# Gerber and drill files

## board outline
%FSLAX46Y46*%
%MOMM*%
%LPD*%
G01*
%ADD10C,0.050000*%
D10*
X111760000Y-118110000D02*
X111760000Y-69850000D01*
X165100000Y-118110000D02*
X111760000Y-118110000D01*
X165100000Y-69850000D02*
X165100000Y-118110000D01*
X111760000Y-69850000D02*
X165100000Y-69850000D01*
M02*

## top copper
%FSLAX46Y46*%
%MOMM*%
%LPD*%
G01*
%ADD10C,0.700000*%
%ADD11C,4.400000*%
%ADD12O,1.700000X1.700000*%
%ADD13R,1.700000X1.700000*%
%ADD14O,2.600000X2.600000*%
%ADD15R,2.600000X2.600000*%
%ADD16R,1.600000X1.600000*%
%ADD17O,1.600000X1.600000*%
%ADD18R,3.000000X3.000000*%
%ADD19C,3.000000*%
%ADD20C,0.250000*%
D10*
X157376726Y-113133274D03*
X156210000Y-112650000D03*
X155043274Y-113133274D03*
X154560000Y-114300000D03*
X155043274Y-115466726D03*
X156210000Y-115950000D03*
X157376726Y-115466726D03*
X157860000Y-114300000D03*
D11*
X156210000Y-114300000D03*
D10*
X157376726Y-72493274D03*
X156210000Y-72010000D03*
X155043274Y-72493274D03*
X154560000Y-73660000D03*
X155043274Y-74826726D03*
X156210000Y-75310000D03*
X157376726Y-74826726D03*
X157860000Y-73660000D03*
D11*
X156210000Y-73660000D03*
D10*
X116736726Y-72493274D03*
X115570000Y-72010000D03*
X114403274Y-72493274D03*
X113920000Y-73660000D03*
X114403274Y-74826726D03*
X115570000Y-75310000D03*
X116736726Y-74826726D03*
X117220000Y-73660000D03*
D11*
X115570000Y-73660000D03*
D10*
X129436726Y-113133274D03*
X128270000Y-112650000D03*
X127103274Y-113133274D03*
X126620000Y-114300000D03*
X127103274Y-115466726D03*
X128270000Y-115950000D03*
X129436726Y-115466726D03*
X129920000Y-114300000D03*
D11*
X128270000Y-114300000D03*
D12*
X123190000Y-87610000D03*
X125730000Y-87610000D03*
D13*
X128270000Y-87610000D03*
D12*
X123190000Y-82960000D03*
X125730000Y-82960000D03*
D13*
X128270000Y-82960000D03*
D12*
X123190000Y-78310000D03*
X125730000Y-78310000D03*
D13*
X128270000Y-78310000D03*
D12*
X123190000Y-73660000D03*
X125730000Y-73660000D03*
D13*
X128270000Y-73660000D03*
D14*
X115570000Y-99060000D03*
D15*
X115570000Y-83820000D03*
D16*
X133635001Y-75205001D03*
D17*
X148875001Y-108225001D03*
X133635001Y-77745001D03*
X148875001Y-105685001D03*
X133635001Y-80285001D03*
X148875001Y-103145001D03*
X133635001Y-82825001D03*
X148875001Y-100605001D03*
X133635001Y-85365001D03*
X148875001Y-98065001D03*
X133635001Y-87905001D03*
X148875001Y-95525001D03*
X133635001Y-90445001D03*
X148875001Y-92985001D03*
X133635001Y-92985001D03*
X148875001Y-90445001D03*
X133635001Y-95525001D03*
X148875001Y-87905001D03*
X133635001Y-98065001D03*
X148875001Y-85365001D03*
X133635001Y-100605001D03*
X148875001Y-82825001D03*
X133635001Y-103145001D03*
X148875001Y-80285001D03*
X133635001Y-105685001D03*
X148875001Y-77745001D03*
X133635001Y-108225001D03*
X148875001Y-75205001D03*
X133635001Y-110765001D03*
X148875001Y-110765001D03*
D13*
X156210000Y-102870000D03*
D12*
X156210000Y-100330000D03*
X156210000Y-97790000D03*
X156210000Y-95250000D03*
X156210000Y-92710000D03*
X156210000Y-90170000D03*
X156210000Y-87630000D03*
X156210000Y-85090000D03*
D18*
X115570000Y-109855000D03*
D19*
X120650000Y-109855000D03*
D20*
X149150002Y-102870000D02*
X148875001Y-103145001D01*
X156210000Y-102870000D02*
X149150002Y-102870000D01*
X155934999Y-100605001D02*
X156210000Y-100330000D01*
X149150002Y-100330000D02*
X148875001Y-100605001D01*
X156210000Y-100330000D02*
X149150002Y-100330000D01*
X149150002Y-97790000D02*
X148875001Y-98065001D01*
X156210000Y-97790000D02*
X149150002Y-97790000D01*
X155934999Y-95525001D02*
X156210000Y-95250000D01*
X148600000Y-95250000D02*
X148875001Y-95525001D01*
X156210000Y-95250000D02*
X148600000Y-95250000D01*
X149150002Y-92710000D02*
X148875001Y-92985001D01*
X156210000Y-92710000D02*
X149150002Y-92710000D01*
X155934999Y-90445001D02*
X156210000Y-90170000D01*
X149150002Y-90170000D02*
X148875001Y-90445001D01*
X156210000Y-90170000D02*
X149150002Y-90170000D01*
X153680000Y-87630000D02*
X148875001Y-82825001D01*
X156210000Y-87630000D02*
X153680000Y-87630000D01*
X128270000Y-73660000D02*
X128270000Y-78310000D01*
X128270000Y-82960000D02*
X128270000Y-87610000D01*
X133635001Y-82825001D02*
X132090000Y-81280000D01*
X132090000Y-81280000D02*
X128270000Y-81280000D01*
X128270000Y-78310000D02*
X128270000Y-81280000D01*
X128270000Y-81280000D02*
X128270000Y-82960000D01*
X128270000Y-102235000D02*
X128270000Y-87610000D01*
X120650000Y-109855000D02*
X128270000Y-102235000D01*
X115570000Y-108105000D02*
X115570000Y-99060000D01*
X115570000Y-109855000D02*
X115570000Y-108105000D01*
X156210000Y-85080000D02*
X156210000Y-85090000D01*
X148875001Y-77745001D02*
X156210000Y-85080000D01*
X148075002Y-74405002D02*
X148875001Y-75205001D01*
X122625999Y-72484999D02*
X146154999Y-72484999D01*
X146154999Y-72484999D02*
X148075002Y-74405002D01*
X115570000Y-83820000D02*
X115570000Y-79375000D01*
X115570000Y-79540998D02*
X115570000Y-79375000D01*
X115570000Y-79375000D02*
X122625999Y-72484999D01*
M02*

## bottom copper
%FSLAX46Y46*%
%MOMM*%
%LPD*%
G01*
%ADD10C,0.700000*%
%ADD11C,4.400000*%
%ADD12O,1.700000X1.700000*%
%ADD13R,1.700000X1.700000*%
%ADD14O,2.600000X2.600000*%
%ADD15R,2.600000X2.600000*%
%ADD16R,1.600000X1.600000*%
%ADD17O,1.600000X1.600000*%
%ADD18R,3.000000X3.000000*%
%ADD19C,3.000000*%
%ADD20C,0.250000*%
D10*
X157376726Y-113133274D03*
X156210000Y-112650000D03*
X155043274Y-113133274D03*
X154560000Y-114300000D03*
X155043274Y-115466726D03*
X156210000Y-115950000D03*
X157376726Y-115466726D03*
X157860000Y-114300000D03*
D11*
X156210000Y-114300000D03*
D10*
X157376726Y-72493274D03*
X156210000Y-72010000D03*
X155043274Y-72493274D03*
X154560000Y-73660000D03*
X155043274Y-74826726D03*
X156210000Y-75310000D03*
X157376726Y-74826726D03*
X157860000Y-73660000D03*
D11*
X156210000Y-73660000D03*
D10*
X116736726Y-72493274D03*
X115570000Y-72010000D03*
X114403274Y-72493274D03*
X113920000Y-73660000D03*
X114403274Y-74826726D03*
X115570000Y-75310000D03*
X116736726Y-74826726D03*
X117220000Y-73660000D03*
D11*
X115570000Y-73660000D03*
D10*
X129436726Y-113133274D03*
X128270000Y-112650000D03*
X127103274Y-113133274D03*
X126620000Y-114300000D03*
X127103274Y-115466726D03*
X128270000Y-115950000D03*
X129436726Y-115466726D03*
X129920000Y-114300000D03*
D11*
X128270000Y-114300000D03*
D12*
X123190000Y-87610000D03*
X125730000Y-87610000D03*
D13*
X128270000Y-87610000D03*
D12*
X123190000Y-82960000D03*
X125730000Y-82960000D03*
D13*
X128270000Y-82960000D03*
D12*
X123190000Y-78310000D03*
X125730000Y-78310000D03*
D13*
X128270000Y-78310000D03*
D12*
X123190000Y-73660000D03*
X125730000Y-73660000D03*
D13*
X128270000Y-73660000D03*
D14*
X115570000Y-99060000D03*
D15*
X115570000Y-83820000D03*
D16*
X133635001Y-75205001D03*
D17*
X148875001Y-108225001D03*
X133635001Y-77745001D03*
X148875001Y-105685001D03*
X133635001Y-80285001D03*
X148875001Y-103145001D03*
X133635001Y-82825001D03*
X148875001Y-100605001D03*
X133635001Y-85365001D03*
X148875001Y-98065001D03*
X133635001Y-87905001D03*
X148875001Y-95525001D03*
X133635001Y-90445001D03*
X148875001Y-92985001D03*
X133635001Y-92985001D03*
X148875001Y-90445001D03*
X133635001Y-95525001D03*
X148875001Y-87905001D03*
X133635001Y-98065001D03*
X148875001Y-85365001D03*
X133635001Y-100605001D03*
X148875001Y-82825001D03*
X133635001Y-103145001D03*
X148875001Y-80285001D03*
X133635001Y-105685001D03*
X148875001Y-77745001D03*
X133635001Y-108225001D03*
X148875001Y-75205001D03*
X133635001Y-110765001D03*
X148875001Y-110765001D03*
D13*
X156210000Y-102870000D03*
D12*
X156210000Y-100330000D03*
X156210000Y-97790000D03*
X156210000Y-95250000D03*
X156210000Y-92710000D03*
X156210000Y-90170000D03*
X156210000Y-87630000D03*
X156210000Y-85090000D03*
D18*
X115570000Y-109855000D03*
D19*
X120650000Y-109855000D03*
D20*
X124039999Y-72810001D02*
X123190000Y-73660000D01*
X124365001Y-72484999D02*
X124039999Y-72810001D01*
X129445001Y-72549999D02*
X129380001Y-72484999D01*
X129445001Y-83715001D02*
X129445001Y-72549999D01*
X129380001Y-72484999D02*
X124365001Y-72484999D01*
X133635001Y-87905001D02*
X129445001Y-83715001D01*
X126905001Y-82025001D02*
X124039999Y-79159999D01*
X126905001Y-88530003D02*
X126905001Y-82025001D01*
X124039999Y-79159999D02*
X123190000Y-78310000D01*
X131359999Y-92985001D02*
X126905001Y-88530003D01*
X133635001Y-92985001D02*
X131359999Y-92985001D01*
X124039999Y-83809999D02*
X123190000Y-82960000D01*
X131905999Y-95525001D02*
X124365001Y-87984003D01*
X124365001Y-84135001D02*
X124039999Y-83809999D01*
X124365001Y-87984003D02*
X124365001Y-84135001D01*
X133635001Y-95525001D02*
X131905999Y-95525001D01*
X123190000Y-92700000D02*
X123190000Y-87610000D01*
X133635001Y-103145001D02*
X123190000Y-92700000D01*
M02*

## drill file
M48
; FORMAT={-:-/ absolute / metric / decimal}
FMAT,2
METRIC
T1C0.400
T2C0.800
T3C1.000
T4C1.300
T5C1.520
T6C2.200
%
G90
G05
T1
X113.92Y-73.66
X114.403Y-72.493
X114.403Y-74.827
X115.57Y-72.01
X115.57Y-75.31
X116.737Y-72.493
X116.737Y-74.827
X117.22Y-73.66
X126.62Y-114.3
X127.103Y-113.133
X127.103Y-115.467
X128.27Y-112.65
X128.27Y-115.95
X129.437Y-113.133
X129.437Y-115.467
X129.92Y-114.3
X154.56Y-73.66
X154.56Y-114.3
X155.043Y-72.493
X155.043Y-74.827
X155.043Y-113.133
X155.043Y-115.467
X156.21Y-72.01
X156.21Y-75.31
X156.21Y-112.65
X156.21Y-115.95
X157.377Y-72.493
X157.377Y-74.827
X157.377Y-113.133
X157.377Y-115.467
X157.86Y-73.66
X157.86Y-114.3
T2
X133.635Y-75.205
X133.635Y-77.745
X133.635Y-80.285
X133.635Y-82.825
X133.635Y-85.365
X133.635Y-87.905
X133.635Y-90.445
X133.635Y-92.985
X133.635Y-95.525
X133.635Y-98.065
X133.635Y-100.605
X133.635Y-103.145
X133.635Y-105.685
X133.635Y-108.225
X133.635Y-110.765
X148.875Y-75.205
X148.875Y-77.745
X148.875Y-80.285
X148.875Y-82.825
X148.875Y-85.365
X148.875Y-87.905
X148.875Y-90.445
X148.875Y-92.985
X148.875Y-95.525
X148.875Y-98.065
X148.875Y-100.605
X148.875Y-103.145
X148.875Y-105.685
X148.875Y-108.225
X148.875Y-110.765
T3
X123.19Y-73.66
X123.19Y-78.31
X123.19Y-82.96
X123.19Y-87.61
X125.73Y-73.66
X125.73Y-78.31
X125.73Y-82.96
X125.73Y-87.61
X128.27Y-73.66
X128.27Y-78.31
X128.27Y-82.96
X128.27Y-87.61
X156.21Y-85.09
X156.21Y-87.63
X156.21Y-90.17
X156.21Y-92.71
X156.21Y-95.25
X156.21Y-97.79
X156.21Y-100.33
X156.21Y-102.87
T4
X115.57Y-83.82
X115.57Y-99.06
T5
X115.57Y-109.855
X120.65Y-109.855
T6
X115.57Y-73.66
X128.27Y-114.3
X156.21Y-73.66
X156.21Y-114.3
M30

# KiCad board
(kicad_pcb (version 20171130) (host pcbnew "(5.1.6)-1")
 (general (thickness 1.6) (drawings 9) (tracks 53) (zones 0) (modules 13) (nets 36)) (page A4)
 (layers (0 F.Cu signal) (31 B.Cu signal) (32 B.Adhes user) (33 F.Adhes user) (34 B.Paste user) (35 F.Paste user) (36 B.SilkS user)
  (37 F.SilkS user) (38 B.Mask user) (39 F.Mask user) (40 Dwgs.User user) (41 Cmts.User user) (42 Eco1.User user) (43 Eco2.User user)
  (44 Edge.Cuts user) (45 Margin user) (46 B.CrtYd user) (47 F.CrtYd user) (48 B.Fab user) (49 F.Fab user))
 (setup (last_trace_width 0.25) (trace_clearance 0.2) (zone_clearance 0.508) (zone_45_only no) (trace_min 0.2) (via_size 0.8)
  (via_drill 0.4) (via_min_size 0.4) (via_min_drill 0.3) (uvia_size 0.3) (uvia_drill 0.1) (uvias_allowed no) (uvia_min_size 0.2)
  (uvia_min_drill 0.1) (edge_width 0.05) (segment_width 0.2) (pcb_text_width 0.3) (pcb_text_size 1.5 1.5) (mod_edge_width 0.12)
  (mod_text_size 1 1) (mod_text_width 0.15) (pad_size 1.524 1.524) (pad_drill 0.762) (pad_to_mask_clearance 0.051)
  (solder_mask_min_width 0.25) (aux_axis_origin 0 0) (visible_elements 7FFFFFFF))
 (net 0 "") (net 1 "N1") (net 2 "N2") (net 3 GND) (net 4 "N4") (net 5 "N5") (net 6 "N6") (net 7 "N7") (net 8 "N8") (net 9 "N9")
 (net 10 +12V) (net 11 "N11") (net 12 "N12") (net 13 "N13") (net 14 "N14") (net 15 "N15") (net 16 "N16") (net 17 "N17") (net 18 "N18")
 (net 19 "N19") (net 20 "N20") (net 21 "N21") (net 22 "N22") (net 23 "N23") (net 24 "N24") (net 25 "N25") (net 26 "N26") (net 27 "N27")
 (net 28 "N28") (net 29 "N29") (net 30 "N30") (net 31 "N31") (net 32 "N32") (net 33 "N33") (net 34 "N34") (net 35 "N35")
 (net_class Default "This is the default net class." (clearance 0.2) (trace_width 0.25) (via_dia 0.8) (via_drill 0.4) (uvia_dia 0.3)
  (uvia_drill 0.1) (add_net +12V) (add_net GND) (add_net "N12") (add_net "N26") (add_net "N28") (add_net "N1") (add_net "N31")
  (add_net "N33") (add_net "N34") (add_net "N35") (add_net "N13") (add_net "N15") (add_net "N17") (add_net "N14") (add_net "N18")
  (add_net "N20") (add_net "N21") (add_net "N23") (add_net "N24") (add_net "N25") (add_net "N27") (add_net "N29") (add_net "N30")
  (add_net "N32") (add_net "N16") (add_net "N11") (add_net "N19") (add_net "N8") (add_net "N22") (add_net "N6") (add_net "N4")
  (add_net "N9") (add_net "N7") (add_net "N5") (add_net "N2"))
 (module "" (layer B.Cu) (at 140.97 92.71 270)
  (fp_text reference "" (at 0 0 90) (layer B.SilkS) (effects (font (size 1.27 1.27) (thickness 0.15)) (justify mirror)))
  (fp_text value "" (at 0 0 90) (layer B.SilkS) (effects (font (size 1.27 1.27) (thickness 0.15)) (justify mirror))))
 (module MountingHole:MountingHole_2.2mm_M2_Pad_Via (layer F.Cu) (at 156.21 114.3)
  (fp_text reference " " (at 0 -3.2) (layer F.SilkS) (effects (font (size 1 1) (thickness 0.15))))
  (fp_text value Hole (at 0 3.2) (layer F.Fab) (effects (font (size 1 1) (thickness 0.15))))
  (pad 1 thru_hole circle (at 1.166726 -1.166726) (size 0.7 0.7) (drill 0.4) (layers *.Cu *.Mask))
  (pad 1 thru_hole circle (at 0 -1.65) (size 0.7 0.7) (drill 0.4) (layers *.Cu *.Mask))
  (pad 1 thru_hole circle (at -1.166726 -1.166726) (size 0.7 0.7) (drill 0.4) (layers *.Cu *.Mask))
  (pad 1 thru_hole circle (at -1.65 0) (size 0.7 0.7) (drill 0.4) (layers *.Cu *.Mask))
  (pad 1 thru_hole circle (at -1.166726 1.166726) (size 0.7 0.7) (drill 0.4) (layers *.Cu *.Mask))
  (pad 1 thru_hole circle (at 0 1.65) (size 0.7 0.7) (drill 0.4) (layers *.Cu *.Mask))
  (pad 1 thru_hole circle (at 1.166726 1.166726) (size 0.7 0.7) (drill 0.4) (layers *.Cu *.Mask))
  (pad 1 thru_hole circle (at 1.65 0) (size 0.7 0.7) (drill 0.4) (layers *.Cu *.Mask))
  (pad 1 thru_hole circle (at 0 0) (size 4.4 4.4) (drill 2.2) (layers *.Cu *.Mask)))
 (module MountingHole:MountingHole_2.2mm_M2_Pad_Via (layer F.Cu) (at 156.21 73.66)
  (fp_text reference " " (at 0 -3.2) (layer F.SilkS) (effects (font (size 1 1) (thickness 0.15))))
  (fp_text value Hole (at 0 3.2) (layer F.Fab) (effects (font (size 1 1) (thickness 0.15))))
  (pad 1 thru_hole circle (at 1.166726 -1.166726) (size 0.7 0.7) (drill 0.4) (layers *.Cu *.Mask))
  (pad 1 thru_hole circle (at 0 -1.65) (size 0.7 0.7) (drill 0.4) (layers *.Cu *.Mask))
  (pad 1 thru_hole circle (at -1.166726 -1.166726) (size 0.7 0.7) (drill 0.4) (layers *.Cu *.Mask))
  (pad 1 thru_hole circle (at -1.65 0) (size 0.7 0.7) (drill 0.4) (layers *.Cu *.Mask))
  (pad 1 thru_hole circle (at -1.166726 1.166726) (size 0.7 0.7) (drill 0.4) (layers *.Cu *.Mask))
  (pad 1 thru_hole circle (at 0 1.65) (size 0.7 0.7) (drill 0.4) (layers *.Cu *.Mask))
  (pad 1 thru_hole circle (at 1.166726 1.166726) (size 0.7 0.7) (drill 0.4) (layers *.Cu *.Mask))
  (pad 1 thru_hole circle (at 1.65 0) (size 0.7 0.7) (drill 0.4) (layers *.Cu *.Mask))
  (pad 1 thru_hole circle (at 0 0) (size 4.4 4.4) (drill 2.2) (layers *.Cu *.Mask)))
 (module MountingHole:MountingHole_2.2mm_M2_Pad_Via (layer F.Cu) (at 115.57 73.66)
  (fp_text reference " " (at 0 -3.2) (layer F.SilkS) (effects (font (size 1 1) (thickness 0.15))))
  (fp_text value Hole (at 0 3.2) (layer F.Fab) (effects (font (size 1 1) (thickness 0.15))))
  (pad 1 thru_hole circle (at 1.166726 -1.166726) (size 0.7 0.7) (drill 0.4) (layers *.Cu *.Mask))
  (pad 1 thru_hole circle (at 0 -1.65) (size 0.7 0.7) (drill 0.4) (layers *.Cu *.Mask))
  (pad 1 thru_hole circle (at -1.166726 -1.166726) (size 0.7 0.7) (drill 0.4) (layers *.Cu *.Mask))
  (pad 1 thru_hole circle (at -1.65 0) (size 0.7 0.7) (drill 0.4) (layers *.Cu *.Mask))
  (pad 1 thru_hole circle (at -1.166726 1.166726) (size 0.7 0.7) (drill 0.4) (layers *.Cu *.Mask))
  (pad 1 thru_hole circle (at 0 1.65) (size 0.7 0.7) (drill 0.4) (layers *.Cu *.Mask))
  (pad 1 thru_hole circle (at 1.166726 1.166726) (size 0.7 0.7) (drill 0.4) (layers *.Cu *.Mask))
  (pad 1 thru_hole circle (at 1.65 0) (size 0.7 0.7) (drill 0.4) (layers *.Cu *.Mask))
  (pad 1 thru_hole circle (at 0 0) (size 4.4 4.4) (drill 2.2) (layers *.Cu *.Mask)))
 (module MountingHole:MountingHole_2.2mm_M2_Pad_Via (layer F.Cu) (at 128.27 114.3)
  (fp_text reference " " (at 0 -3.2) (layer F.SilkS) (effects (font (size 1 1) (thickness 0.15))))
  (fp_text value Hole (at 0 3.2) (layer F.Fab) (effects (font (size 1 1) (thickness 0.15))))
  (pad 1 thru_hole circle (at 1.166726 -1.166726) (size 0.7 0.7) (drill 0.4) (layers *.Cu *.Mask))
  (pad 1 thru_hole circle (at 0 -1.65) (size 0.7 0.7) (drill 0.4) (layers *.Cu *.Mask))
  (pad 1 thru_hole circle (at -1.166726 -1.166726) (size 0.7 0.7) (drill 0.4) (layers *.Cu *.Mask))
  (pad 1 thru_hole circle (at -1.65 0) (size 0.7 0.7) (drill 0.4) (layers *.Cu *.Mask))
  (pad 1 thru_hole circle (at -1.166726 1.166726) (size 0.7 0.7) (drill 0.4) (layers *.Cu *.Mask))
  (pad 1 thru_hole circle (at 0 1.65) (size 0.7 0.7) (drill 0.4) (layers *.Cu *.Mask))
  (pad 1 thru_hole circle (at 1.166726 1.166726) (size 0.7 0.7) (drill 0.4) (layers *.Cu *.Mask))
  (pad 1 thru_hole circle (at 1.65 0) (size 0.7 0.7) (drill 0.4) (layers *.Cu *.Mask))
  (pad 1 thru_hole circle (at 0 0) (size 4.4 4.4) (drill 2.2) (layers *.Cu *.Mask)))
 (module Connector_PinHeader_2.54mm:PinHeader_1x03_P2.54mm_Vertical (layer F.Cu) (at 128.27 87.61 270)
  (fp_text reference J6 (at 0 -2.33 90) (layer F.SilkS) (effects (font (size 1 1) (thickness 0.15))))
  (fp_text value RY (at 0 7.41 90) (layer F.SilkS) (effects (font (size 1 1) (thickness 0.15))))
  (pad 3 thru_hole oval (at 0 5.08 270) (size 1.7 1.7) (drill 1) (layers *.Cu *.Mask) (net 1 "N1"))
  (pad 2 thru_hole oval (at 0 2.54 270) (size 1.7 1.7) (drill 1) (layers *.Cu *.Mask) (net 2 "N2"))
  (pad 1 thru_hole rect (at 0 0 270) (size 1.7 1.7) (drill 1) (layers *.Cu *.Mask) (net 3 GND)))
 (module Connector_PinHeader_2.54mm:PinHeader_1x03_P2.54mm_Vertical (layer F.Cu) (at 128.27 82.96 270)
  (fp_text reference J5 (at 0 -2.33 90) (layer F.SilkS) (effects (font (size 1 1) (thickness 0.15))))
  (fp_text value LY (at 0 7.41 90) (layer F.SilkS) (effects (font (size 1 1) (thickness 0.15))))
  (pad 3 thru_hole oval (at 0 5.08 270) (size 1.7 1.7) (drill 1) (layers *.Cu *.Mask) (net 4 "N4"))
  (pad 2 thru_hole oval (at 0 2.54 270) (size 1.7 1.7) (drill 1) (layers *.Cu *.Mask) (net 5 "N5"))
  (pad 1 thru_hole rect (at 0 0 270) (size 1.7 1.7) (drill 1) (layers *.Cu *.Mask) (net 3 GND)))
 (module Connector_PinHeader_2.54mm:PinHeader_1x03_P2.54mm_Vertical (layer F.Cu) (at 128.27 78.31 270)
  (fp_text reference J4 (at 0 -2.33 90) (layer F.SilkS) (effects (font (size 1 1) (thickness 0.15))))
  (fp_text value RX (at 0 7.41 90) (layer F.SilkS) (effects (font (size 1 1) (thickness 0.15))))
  (pad 3 thru_hole oval (at 0 5.08 270) (size 1.7 1.7) (drill 1) (layers *.Cu *.Mask) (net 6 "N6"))
  (pad 2 thru_hole oval (at 0 2.54 270) (size 1.7 1.7) (drill 1) (layers *.Cu *.Mask) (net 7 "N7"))
  (pad 1 thru_hole rect (at 0 0 270) (size 1.7 1.7) (drill 1) (layers *.Cu *.Mask) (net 3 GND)))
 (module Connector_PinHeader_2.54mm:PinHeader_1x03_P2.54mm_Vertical (layer F.Cu) (at 128.27 73.66 270)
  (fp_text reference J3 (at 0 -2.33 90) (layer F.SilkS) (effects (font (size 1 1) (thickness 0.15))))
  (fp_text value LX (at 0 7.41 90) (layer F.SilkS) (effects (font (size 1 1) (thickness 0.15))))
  (pad 3 thru_hole oval (at 0 5.08 270) (size 1.7 1.7) (drill 1) (layers *.Cu *.Mask) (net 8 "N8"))
  (pad 2 thru_hole oval (at 0 2.54 270) (size 1.7 1.7) (drill 1) (layers *.Cu *.Mask) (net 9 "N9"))
  (pad 1 thru_hole rect (at 0 0 270) (size 1.7 1.7) (drill 1) (layers *.Cu *.Mask) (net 3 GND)))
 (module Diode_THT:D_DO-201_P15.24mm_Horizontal (layer F.Cu) (at 115.57 83.82 270)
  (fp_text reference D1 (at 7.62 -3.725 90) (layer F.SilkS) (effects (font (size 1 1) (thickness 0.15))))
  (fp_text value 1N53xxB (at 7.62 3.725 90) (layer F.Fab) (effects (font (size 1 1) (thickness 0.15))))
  (pad 2 thru_hole oval (at 15.24 0 270) (size 2.6 2.6) (drill 1.3) (layers *.Cu *.Mask) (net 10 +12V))
  (pad 1 thru_hole rect (at 0 0 270) (size 2.6 2.6) (drill 1.3) (layers *.Cu *.Mask) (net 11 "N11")))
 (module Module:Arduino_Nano (layer F.Cu) (at 133.635001 75.205001)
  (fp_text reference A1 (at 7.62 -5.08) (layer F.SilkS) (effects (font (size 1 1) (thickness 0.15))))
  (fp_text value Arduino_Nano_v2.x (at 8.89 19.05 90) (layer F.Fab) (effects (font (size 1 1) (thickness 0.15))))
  (pad 1 thru_hole rect (at 0 0) (size 1.6 1.6) (drill 0.8) (layers *.Cu *.Mask) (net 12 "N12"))
  (pad 17 thru_hole oval (at 15.24 33.02) (size 1.6 1.6) (drill 0.8) (layers *.Cu *.Mask) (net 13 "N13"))
  (pad 2 thru_hole oval (at 0 2.54) (size 1.6 1.6) (drill 0.8) (layers *.Cu *.Mask) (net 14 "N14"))
  (pad 18 thru_hole oval (at 15.24 30.48) (size 1.6 1.6) (drill 0.8) (layers *.Cu *.Mask) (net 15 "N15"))
  (pad 3 thru_hole oval (at 0 5.08) (size 1.6 1.6) (drill 0.8) (layers *.Cu *.Mask) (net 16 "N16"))
  (pad 19 thru_hole oval (at 15.24 27.94) (size 1.6 1.6) (drill 0.8) (layers *.Cu *.Mask) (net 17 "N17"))
  (pad 4 thru_hole oval (at 0 7.62) (size 1.6 1.6) (drill 0.8) (layers *.Cu *.Mask) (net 3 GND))
  (pad 20 thru_hole oval (at 15.24 25.4) (size 1.6 1.6) (drill 0.8) (layers *.Cu *.Mask) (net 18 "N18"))
  (pad 5 thru_hole oval (at 0 10.16) (size 1.6 1.6) (drill 0.8) (layers *.Cu *.Mask) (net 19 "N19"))
  (pad 21 thru_hole oval (at 15.24 22.86) (size 1.6 1.6) (drill 0.8) (layers *.Cu *.Mask) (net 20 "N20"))
  (pad 6 thru_hole oval (at 0 12.7) (size 1.6 1.6) (drill 0.8) (layers *.Cu *.Mask) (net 8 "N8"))
  (pad 22 thru_hole oval (at 15.24 20.32) (size 1.6 1.6) (drill 0.8) (layers *.Cu *.Mask) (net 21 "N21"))
  (pad 7 thru_hole oval (at 0 15.24) (size 1.6 1.6) (drill 0.8) (layers *.Cu *.Mask) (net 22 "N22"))
  (pad 23 thru_hole oval (at 15.24 17.78) (size 1.6 1.6) (drill 0.8) (layers *.Cu *.Mask) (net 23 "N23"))
  (pad 8 thru_hole oval (at 0 17.78) (size 1.6 1.6) (drill 0.8) (layers *.Cu *.Mask) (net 6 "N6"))
  (pad 24 thru_hole oval (at 15.24 15.24) (size 1.6 1.6) (drill 0.8) (layers *.Cu *.Mask) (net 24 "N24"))
  (pad 9 thru_hole oval (at 0 20.32) (size 1.6 1.6) (drill 0.8) (layers *.Cu *.Mask) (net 4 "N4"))
  (pad 25 thru_hole oval (at 15.24 12.7) (size 1.6 1.6) (drill 0.8) (layers *.Cu *.Mask) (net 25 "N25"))
  (pad 10 thru_hole oval (at 0 22.86) (size 1.6 1.6) (drill 0.8) (layers *.Cu *.Mask) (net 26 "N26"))
  (pad 26 thru_hole oval (at 15.24 10.16) (size 1.6 1.6) (drill 0.8) (layers *.Cu *.Mask) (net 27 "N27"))
  (pad 11 thru_hole oval (at 0 25.4) (size 1.6 1.6) (drill 0.8) (layers *.Cu *.Mask) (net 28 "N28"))
  (pad 27 thru_hole oval (at 15.24 7.62) (size 1.6 1.6) (drill 0.8) (layers *.Cu *.Mask) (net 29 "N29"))
  (pad 12 thru_hole oval (at 0 27.94) (size 1.6 1.6) (drill 0.8) (layers *.Cu *.Mask) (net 1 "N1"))
  (pad 28 thru_hole oval (at 15.24 5.08) (size 1.6 1.6) (drill 0.8) (layers *.Cu *.Mask) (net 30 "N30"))
  (pad 13 thru_hole oval (at 0 30.48) (size 1.6 1.6) (drill 0.8) (layers *.Cu *.Mask) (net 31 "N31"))
  (pad 29 thru_hole oval (at 15.24 2.54) (size 1.6 1.6) (drill 0.8) (layers *.Cu *.Mask) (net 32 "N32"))
  (pad 14 thru_hole oval (at 0 33.02) (size 1.6 1.6) (drill 0.8) (layers *.Cu *.Mask) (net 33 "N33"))
  (pad 30 thru_hole oval (at 15.24 0) (size 1.6 1.6) (drill 0.8) (layers *.Cu *.Mask) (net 11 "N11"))
  (pad 15 thru_hole oval (at 0 35.56) (size 1.6 1.6) (drill 0.8) (layers *.Cu *.Mask) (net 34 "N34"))
  (pad 16 thru_hole oval (at 15.24 35.56) (size 1.6 1.6) (drill 0.8) (layers *.Cu *.Mask) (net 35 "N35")))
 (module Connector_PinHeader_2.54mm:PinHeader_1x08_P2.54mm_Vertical (layer F.Cu) (at 156.21 102.87 180)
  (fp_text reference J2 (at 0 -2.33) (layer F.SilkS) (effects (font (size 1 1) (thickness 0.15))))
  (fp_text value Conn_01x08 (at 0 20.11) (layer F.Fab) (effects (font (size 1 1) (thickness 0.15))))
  (pad 1 thru_hole rect (at 0 0 180) (size 1.7 1.7) (drill 1) (layers *.Cu *.Mask) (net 17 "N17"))
  (pad 2 thru_hole oval (at 0 2.54 180) (size 1.7 1.7) (drill 1) (layers *.Cu *.Mask) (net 18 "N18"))
  (pad 3 thru_hole oval (at 0 5.08 180) (size 1.7 1.7) (drill 1) (layers *.Cu *.Mask) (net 20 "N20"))
  (pad 4 thru_hole oval (at 0 7.62 180) (size 1.7 1.7) (drill 1) (layers *.Cu *.Mask) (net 21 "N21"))
  (pad 5 thru_hole oval (at 0 10.16 180) (size 1.7 1.7) (drill 1) (layers *.Cu *.Mask) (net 23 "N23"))
  (pad 6 thru_hole oval (at 0 12.7 180) (size 1.7 1.7) (drill 1) (layers *.Cu *.Mask) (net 24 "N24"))
  (pad 7 thru_hole oval (at 0 15.24 180) (size 1.7 1.7) (drill 1) (layers *.Cu *.Mask) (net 29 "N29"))
  (pad 8 thru_hole oval (at 0 17.78 180) (size 1.7 1.7) (drill 1) (layers *.Cu *.Mask) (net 32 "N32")))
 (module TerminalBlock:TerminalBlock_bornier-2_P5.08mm (layer F.Cu) (at 115.57 109.855)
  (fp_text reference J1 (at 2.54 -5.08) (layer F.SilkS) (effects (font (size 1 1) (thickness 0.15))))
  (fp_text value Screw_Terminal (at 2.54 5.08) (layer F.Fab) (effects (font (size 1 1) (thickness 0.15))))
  (pad 1 thru_hole rect (at 0 0) (size 3 3) (drill 1.52) (layers *.Cu *.Mask) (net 10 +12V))
  (pad 2 thru_hole circle (at 5.08 0) (size 3 3) (drill 1.52) (layers *.Cu *.Mask) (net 3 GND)))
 (gr_line (start 111.76 118.11) (end 111.76 69.85) (layer Edge.Cuts) (width 0.05))
 (gr_line (start 165.1 118.11) (end 111.76 118.11) (layer Edge.Cuts) (width 0.05))
 (gr_line (start 165.1 69.85) (end 165.1 118.11) (layer Edge.Cuts) (width 0.05))
 (gr_line (start 111.76 69.85) (end 165.1 69.85) (layer Edge.Cuts) (width 0.05))
 (segment (start 149.150002 102.87) (end 148.875001 103.145001) (width 0.25) (layer F.Cu) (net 17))
 (segment (start 156.21 102.87) (end 149.150002 102.87) (width 0.25) (layer F.Cu) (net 17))
 (segment (start 155.934999 100.605001) (end 156.21 100.33) (width 0.25) (layer F.Cu) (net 18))
 (segment (start 149.150002 100.33) (end 148.875001 100.605001) (width 0.25) (layer F.Cu) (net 18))
 (segment (start 156.21 100.33) (end 149.150002 100.33) (width 0.25) (layer F.Cu) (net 18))
 (segment (start 149.150002 97.79) (end 148.875001 98.065001) (width 0.25) (layer F.Cu) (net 20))
 (segment (start 156.21 97.79) (end 149.150002 97.79) (width 0.25) (layer F.Cu) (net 20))
 (segment (start 124.039999 72.810001) (end 123.19 73.66) (width 0.25) (layer B.Cu) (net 8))
 (segment (start 124.365001 72.484999) (end 124.039999 72.810001) (width 0.25) (layer B.Cu) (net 8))
 (segment (start 129.445001 72.549999) (end 129.380001 72.484999) (width 0.25) (layer B.Cu) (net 8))
 (segment (start 129.445001 83.715001) (end 129.445001 72.549999) (width 0.25) (layer B.Cu) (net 8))
 (segment (start 129.380001 72.484999) (end 124.365001 72.484999) (width 0.25) (layer B.Cu) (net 8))
 (segment (start 133.635001 87.905001) (end 129.445001 83.715001) (width 0.25) (layer B.Cu) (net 8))
 (segment (start 155.934999 95.525001) (end 156.21 95.25) (width 0.25) (layer F.Cu) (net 21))
 (segment (start 148.6 95.25) (end 148.875001 95.525001) (width 0.25) (layer F.Cu) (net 21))
 (segment (start 156.21 95.25) (end 148.6 95.25) (width 0.25) (layer F.Cu) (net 21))
 (segment (start 149.150002 92.71) (end 148.875001 92.985001) (width 0.25) (layer F.Cu) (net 23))
 (segment (start 156.21 92.71) (end 149.150002 92.71) (width 0.25) (layer F.Cu) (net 23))
 (segment (start 126.905001 82.025001) (end 124.039999 79.159999) (width 0.25) (layer B.Cu) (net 6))
 (segment (start 126.905001 88.530003) (end 126.905001 82.025001) (width 0.25) (layer B.Cu) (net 6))
 (segment (start 124.039999 79.159999) (end 123.19 78.31) (width 0.25) (layer B.Cu) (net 6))
 (segment (start 131.359999 92.985001) (end 126.905001 88.530003) (width 0.25) (layer B.Cu) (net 6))
 (segment (start 133.635001 92.985001) (end 131.359999 92.985001) (width 0.25) (layer B.Cu) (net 6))
 (segment (start 155.934999 90.445001) (end 156.21 90.17) (width 0.25) (layer F.Cu) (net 24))
 (segment (start 149.150002 90.17) (end 148.875001 90.445001) (width 0.25) (layer F.Cu) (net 24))
 (segment (start 156.21 90.17) (end 149.150002 90.17) (width 0.25) (layer F.Cu) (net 24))
 (segment (start 124.039999 83.809999) (end 123.19 82.96) (width 0.25) (layer B.Cu) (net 4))
 (segment (start 131.905999 95.525001) (end 124.365001 87.984003) (width 0.25) (layer B.Cu) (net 4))
 (segment (start 124.365001 84.135001) (end 124.039999 83.809999) (width 0.25) (layer B.Cu) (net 4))
 (segment (start 124.365001 87.984003) (end 124.365001 84.135001) (width 0.25) (layer B.Cu) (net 4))
 (segment (start 133.635001 95.525001) (end 131.905999 95.525001) (width 0.25) (layer B.Cu) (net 4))
 (segment (start 153.68 87.63) (end 148.875001 82.825001) (width 0.25) (layer F.Cu) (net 29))
 (segment (start 156.21 87.63) (end 153.68 87.63) (width 0.25) (layer F.Cu) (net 29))
 (segment (start 123.19 92.7) (end 123.19 87.61) (width 0.25) (layer B.Cu) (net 1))
 (segment (start 133.635001 103.145001) (end 123.19 92.7) (width 0.25) (layer B.Cu) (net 1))
 (segment (start 128.27 73.66) (end 128.27 78.31) (width 0.25) (layer F.Cu) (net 3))
 (segment (start 128.27 82.96) (end 128.27 87.61) (width 0.25) (layer F.Cu) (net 3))
 (segment (start 133.635001 82.825001) (end 132.09 81.28) (width 0.25) (layer F.Cu) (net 3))
 (segment (start 132.09 81.28) (end 128.27 81.28) (width 0.25) (layer F.Cu) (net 3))
 (segment (start 128.27 78.31) (end 128.27 81.28) (width 0.25) (layer F.Cu) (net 3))
 (segment (start 128.27 81.28) (end 128.27 82.96) (width 0.25) (layer F.Cu) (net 3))
 (segment (start 128.27 102.235) (end 128.27 87.61) (width 0.25) (layer F.Cu) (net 3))
 (segment (start 120.65 109.855) (end 128.27 102.235) (width 0.25) (layer F.Cu) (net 3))
 (segment (start 115.57 108.105) (end 115.57 99.06) (width 0.25) (layer F.Cu) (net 10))
 (segment (start 115.57 109.855) (end 115.57 108.105) (width 0.25) (layer F.Cu) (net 10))
 (segment (start 156.21 85.08) (end 156.21 85.09) (width 0.25) (layer F.Cu) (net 32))
 (segment (start 148.875001 77.745001) (end 156.21 85.08) (width 0.25) (layer F.Cu) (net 32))
 (segment (start 148.075002 74.405002) (end 148.875001 75.205001) (width 0.25) (layer F.Cu) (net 11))
 (segment (start 122.625999 72.484999) (end 146.154999 72.484999) (width 0.25) (layer F.Cu) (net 11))
 (segment (start 146.154999 72.484999) (end 148.075002 74.405002) (width 0.25) (layer F.Cu) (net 11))
 (segment (start 115.57 83.82) (end 115.57 79.375) (width 0.25) (layer F.Cu) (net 11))
 (segment (start 115.57 79.540998) (end 115.57 79.375) (width 0.25) (layer F.Cu) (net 11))
 (segment (start 115.57 79.375) (end 122.625999 72.484999) (width 0.25) (layer F.Cu) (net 11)))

